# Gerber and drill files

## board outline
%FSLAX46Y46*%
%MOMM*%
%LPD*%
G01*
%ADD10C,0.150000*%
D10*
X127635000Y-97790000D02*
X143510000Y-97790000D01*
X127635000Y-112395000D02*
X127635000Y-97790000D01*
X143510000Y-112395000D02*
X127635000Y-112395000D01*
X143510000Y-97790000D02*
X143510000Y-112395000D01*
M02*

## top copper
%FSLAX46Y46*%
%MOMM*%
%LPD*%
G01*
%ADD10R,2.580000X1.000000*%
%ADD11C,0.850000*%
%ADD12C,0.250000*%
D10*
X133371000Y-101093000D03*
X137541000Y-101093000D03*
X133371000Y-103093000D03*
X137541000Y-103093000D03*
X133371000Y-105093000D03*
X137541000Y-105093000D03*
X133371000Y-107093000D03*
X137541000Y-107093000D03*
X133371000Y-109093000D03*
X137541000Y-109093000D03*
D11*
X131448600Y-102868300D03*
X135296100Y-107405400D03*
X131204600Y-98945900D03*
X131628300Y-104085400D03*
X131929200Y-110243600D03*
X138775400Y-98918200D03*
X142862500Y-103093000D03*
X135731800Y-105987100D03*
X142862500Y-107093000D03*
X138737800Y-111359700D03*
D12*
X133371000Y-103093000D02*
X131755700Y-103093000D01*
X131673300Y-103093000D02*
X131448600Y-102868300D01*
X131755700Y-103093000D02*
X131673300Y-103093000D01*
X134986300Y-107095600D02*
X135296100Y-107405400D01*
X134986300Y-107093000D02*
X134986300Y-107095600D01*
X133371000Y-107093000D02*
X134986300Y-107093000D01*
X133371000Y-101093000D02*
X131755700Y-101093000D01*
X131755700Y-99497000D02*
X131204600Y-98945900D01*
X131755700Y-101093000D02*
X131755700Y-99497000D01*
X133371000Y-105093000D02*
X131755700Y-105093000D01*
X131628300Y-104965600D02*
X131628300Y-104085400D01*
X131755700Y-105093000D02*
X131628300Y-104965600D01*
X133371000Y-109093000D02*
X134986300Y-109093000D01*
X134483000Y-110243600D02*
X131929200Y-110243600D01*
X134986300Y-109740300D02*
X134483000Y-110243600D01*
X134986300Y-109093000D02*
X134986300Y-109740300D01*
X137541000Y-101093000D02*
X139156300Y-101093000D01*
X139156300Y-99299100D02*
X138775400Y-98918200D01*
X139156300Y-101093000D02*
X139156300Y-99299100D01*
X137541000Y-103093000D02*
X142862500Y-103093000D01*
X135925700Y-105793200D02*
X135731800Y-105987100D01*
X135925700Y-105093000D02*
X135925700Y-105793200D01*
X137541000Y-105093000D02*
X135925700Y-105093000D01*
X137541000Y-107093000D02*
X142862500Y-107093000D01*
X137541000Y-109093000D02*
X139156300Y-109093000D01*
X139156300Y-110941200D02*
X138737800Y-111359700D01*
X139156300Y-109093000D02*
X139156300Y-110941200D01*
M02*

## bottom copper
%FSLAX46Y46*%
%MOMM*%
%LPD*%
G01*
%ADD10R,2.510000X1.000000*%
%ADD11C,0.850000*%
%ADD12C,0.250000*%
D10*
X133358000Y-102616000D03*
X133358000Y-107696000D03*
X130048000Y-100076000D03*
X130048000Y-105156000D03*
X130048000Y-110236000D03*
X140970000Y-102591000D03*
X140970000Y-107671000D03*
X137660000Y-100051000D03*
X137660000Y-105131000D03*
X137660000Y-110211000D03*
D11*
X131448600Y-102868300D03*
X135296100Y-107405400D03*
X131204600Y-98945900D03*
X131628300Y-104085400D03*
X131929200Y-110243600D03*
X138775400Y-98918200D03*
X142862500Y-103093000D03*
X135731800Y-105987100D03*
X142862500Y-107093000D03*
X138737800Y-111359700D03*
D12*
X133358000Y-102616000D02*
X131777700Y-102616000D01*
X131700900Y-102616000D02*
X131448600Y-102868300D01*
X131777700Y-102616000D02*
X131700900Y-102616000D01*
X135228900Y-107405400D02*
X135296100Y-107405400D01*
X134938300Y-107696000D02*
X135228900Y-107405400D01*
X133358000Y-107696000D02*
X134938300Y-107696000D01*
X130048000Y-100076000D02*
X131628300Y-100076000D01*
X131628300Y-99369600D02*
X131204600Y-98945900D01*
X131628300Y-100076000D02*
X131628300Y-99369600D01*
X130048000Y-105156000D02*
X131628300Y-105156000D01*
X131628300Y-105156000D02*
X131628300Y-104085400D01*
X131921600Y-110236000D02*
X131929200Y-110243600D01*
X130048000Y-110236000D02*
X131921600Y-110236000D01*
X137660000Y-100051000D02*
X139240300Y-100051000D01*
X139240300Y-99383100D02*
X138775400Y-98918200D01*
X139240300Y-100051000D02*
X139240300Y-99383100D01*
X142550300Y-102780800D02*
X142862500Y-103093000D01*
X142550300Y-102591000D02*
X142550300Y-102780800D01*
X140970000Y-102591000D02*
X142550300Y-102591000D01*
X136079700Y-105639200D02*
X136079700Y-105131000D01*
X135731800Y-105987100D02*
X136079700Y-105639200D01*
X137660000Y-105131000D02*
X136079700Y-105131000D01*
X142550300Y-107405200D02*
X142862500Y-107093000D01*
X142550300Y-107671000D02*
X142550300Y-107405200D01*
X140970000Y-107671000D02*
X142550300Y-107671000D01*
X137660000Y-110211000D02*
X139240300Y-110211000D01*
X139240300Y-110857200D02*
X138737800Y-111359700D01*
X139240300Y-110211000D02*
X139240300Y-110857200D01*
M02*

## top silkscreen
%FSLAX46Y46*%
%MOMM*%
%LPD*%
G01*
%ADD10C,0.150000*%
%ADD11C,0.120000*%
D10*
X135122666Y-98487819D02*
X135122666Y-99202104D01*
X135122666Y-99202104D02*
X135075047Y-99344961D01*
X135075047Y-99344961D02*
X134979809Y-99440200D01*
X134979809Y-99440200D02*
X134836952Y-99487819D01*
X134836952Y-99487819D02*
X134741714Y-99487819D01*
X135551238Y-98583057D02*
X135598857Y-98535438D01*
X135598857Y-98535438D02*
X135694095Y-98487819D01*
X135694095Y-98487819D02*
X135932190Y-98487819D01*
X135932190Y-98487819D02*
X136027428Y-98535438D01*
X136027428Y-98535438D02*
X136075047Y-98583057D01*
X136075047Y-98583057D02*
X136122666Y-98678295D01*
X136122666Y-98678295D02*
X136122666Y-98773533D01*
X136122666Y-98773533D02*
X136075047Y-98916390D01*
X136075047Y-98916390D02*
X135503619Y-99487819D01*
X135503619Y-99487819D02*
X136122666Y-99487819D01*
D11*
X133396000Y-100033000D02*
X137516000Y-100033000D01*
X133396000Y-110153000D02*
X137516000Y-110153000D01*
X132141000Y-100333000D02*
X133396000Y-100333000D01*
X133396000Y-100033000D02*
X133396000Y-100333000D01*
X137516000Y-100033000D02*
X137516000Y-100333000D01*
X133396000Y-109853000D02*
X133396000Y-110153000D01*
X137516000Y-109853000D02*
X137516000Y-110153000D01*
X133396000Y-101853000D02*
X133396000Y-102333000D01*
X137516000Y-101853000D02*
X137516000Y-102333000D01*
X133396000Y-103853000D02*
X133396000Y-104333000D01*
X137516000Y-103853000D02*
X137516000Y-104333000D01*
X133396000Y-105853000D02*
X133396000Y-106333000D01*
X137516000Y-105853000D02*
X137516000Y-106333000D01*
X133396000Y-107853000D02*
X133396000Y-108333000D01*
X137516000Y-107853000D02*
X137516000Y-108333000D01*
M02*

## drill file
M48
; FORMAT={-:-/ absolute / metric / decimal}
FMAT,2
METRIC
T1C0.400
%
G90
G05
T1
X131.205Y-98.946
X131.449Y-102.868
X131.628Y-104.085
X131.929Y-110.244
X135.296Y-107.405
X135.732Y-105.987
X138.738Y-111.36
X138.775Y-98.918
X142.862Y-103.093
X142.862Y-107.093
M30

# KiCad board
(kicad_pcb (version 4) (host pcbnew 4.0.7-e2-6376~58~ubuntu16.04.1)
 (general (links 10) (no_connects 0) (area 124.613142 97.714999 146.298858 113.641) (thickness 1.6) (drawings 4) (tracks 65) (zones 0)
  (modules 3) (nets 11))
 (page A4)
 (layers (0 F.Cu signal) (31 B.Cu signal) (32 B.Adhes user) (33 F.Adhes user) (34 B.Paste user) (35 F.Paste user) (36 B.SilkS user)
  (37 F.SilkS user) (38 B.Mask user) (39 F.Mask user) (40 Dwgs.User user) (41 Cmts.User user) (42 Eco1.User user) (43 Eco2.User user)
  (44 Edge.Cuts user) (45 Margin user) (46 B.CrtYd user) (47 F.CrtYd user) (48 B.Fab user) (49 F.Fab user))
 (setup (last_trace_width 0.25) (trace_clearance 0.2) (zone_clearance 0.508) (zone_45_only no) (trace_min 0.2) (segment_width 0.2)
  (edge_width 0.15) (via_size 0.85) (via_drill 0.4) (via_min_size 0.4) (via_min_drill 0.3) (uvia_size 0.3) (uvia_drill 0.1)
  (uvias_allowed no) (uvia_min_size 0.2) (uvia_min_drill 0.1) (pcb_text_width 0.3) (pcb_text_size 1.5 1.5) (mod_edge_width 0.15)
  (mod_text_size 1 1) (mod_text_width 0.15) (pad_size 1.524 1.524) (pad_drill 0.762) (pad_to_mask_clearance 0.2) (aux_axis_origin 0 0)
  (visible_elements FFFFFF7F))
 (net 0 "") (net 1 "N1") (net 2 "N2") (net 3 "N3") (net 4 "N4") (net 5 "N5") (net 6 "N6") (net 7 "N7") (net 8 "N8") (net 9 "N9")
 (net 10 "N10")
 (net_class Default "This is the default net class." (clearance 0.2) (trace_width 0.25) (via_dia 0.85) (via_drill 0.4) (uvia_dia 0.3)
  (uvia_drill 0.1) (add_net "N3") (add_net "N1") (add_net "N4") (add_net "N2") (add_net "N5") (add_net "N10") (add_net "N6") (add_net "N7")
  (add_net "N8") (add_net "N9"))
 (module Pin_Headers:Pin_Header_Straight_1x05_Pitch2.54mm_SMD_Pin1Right (layer B.Cu) (at 131.703 105.156 180)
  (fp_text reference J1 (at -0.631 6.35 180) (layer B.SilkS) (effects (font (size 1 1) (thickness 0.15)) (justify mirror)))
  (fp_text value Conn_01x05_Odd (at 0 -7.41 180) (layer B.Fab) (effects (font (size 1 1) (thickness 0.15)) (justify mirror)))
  (pad 2 smd rect (at -1.655 2.54 180) (size 2.51 1) (layers B.Cu B.Paste B.Mask) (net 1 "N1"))
  (pad 4 smd rect (at -1.655 -2.54 180) (size 2.51 1) (layers B.Cu B.Paste B.Mask) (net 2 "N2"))
  (pad 1 smd rect (at 1.655 5.08 180) (size 2.51 1) (layers B.Cu B.Paste B.Mask) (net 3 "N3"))
  (pad 3 smd rect (at 1.655 0 180) (size 2.51 1) (layers B.Cu B.Paste B.Mask) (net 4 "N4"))
  (pad 5 smd rect (at 1.655 -5.08 180) (size 2.51 1) (layers B.Cu B.Paste B.Mask) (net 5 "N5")))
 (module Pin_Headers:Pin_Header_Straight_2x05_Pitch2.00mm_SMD (layer F.Cu) (at 135.456 105.093)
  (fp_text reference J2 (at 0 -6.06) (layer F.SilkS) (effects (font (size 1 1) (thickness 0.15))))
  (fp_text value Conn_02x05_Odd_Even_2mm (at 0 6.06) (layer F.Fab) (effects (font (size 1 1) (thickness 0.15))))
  (fp_line (start -2.06 -5.06) (end 2.06 -5.06) (layer F.SilkS) (width 0.12))
  (fp_line (start -2.06 5.06) (end 2.06 5.06) (layer F.SilkS) (width 0.12))
  (fp_line (start -3.315 -4.76) (end -2.06 -4.76) (layer F.SilkS) (width 0.12))
  (fp_line (start -2.06 -5.06) (end -2.06 -4.76) (layer F.SilkS) (width 0.12))
  (fp_line (start 2.06 -5.06) (end 2.06 -4.76) (layer F.SilkS) (width 0.12))
  (fp_line (start -2.06 4.76) (end -2.06 5.06) (layer F.SilkS) (width 0.12))
  (fp_line (start 2.06 4.76) (end 2.06 5.06) (layer F.SilkS) (width 0.12))
  (fp_line (start -2.06 -3.24) (end -2.06 -2.76) (layer F.SilkS) (width 0.12))
  (fp_line (start 2.06 -3.24) (end 2.06 -2.76) (layer F.SilkS) (width 0.12))
  (fp_line (start -2.06 -1.24) (end -2.06 -0.76) (layer F.SilkS) (width 0.12))
  (fp_line (start 2.06 -1.24) (end 2.06 -0.76) (layer F.SilkS) (width 0.12))
  (fp_line (start -2.06 0.76) (end -2.06 1.24) (layer F.SilkS) (width 0.12))
  (fp_line (start 2.06 0.76) (end 2.06 1.24) (layer F.SilkS) (width 0.12))
  (fp_line (start -2.06 2.76) (end -2.06 3.24) (layer F.SilkS) (width 0.12))
  (fp_line (start 2.06 2.76) (end 2.06 3.24) (layer F.SilkS) (width 0.12))
  (pad 1 smd rect (at -2.085 -4) (size 2.58 1) (layers F.Cu F.Paste F.Mask) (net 3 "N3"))
  (pad 2 smd rect (at 2.085 -4) (size 2.58 1) (layers F.Cu F.Paste F.Mask) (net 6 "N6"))
  (pad 3 smd rect (at -2.085 -2) (size 2.58 1) (layers F.Cu F.Paste F.Mask) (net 1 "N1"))
  (pad 4 smd rect (at 2.085 -2) (size 2.58 1) (layers F.Cu F.Paste F.Mask) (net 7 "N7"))
  (pad 5 smd rect (at -2.085 0) (size 2.58 1) (layers F.Cu F.Paste F.Mask) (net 4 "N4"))
  (pad 6 smd rect (at 2.085 0) (size 2.58 1) (layers F.Cu F.Paste F.Mask) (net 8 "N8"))
  (pad 7 smd rect (at -2.085 2) (size 2.58 1) (layers F.Cu F.Paste F.Mask) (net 2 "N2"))
  (pad 8 smd rect (at 2.085 2) (size 2.58 1) (layers F.Cu F.Paste F.Mask) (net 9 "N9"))
  (pad 9 smd rect (at -2.085 4) (size 2.58 1) (layers F.Cu F.Paste F.Mask) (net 5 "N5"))
  (pad 10 smd rect (at 2.085 4) (size 2.58 1) (layers F.Cu F.Paste F.Mask) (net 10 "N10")))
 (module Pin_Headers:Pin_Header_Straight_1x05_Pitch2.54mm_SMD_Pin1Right (layer B.Cu) (at 139.315 105.131 180)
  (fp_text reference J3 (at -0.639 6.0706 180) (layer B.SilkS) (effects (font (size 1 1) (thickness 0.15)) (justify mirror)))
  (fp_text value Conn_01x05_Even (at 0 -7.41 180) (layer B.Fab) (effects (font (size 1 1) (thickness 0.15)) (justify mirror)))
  (pad 2 smd rect (at -1.655 2.54 180) (size 2.51 1) (layers B.Cu B.Paste B.Mask) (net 7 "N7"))
  (pad 4 smd rect (at -1.655 -2.54 180) (size 2.51 1) (layers B.Cu B.Paste B.Mask) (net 9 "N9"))
  (pad 1 smd rect (at 1.655 5.08 180) (size 2.51 1) (layers B.Cu B.Paste B.Mask) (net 6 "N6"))
  (pad 3 smd rect (at 1.655 0 180) (size 2.51 1) (layers B.Cu B.Paste B.Mask) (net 8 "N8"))
  (pad 5 smd rect (at 1.655 -5.08 180) (size 2.51 1) (layers B.Cu B.Paste B.Mask) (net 10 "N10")))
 (gr_line (start 127.635 97.79) (end 143.51 97.79) (layer Edge.Cuts) (width 0.15))
 (gr_line (start 127.635 112.395) (end 127.635 97.79) (layer Edge.Cuts) (width 0.15))
 (gr_line (start 143.51 112.395) (end 127.635 112.395) (layer Edge.Cuts) (width 0.15))
 (gr_line (start 143.51 97.79) (end 143.51 112.395) (layer Edge.Cuts) (width 0.15))
 (via (at 131.4486 102.8683) (size 0.85) (layers F.Cu B.Cu) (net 1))
 (segment (start 133.358 102.616) (end 131.7777 102.616) (width 0.25) (layer B.Cu) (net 1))
 (segment (start 133.371 103.093) (end 131.7557 103.093) (width 0.25) (layer F.Cu) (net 1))
 (segment (start 131.7009 102.616) (end 131.4486 102.8683) (width 0.25) (layer B.Cu) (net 1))
 (segment (start 131.7777 102.616) (end 131.7009 102.616) (width 0.25) (layer B.Cu) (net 1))
 (segment (start 131.6733 103.093) (end 131.4486 102.8683) (width 0.25) (layer F.Cu) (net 1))
 (segment (start 131.7557 103.093) (end 131.6733 103.093) (width 0.25) (layer F.Cu) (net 1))
 (via (at 135.2961 107.4054) (size 0.85) (layers F.Cu B.Cu) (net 2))
 (segment (start 135.2289 107.4054) (end 135.2961 107.4054) (width 0.25) (layer B.Cu) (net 2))
 (segment (start 134.9383 107.696) (end 135.2289 107.4054) (width 0.25) (layer B.Cu) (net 2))
 (segment (start 134.9863 107.0956) (end 135.2961 107.4054) (width 0.25) (layer F.Cu) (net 2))
 (segment (start 134.9863 107.093) (end 134.9863 107.0956) (width 0.25) (layer F.Cu) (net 2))
 (segment (start 133.371 107.093) (end 134.9863 107.093) (width 0.25) (layer F.Cu) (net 2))
 (segment (start 133.358 107.696) (end 134.9383 107.696) (width 0.25) (layer B.Cu) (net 2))
 (via (at 131.2046 98.9459) (size 0.85) (layers F.Cu B.Cu) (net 3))
 (segment (start 133.371 101.093) (end 131.7557 101.093) (width 0.25) (layer F.Cu) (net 3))
 (segment (start 130.048 100.076) (end 131.6283 100.076) (width 0.25) (layer B.Cu) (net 3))
 (segment (start 131.6283 99.3696) (end 131.2046 98.9459) (width 0.25) (layer B.Cu) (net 3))
 (segment (start 131.6283 100.076) (end 131.6283 99.3696) (width 0.25) (layer B.Cu) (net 3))
 (segment (start 131.7557 99.497) (end 131.2046 98.9459) (width 0.25) (layer F.Cu) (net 3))
 (segment (start 131.7557 101.093) (end 131.7557 99.497) (width 0.25) (layer F.Cu) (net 3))
 (via (at 131.6283 104.0854) (size 0.85) (layers F.Cu B.Cu) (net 4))
 (segment (start 133.371 105.093) (end 131.7557 105.093) (width 0.25) (layer F.Cu) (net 4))
 (segment (start 130.048 105.156) (end 131.6283 105.156) (width 0.25) (layer B.Cu) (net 4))
 (segment (start 131.6283 105.156) (end 131.6283 104.0854) (width 0.25) (layer B.Cu) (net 4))
 (segment (start 131.6283 104.9656) (end 131.6283 104.0854) (width 0.25) (layer F.Cu) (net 4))
 (segment (start 131.7557 105.093) (end 131.6283 104.9656) (width 0.25) (layer F.Cu) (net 4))
 (via (at 131.9292 110.2436) (size 0.85) (layers F.Cu B.Cu) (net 5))
 (segment (start 133.371 109.093) (end 134.9863 109.093) (width 0.25) (layer F.Cu) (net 5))
 (segment (start 131.9216 110.236) (end 131.9292 110.2436) (width 0.25) (layer B.Cu) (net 5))
 (segment (start 130.048 110.236) (end 131.9216 110.236) (width 0.25) (layer B.Cu) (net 5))
 (segment (start 134.483 110.2436) (end 131.9292 110.2436) (width 0.25) (layer F.Cu) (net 5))
 (segment (start 134.9863 109.7403) (end 134.483 110.2436) (width 0.25) (layer F.Cu) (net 5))
 (segment (start 134.9863 109.093) (end 134.9863 109.7403) (width 0.25) (layer F.Cu) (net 5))
 (via (at 138.7754 98.9182) (size 0.85) (layers F.Cu B.Cu) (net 6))
 (segment (start 137.541 101.093) (end 139.1563 101.093) (width 0.25) (layer F.Cu) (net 6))
 (segment (start 137.66 100.051) (end 139.2403 100.051) (width 0.25) (layer B.Cu) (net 6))
 (segment (start 139.2403 99.3831) (end 138.7754 98.9182) (width 0.25) (layer B.Cu) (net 6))
 (segment (start 139.2403 100.051) (end 139.2403 99.3831) (width 0.25) (layer B.Cu) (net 6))
 (segment (start 139.1563 99.2991) (end 138.7754 98.9182) (width 0.25) (layer F.Cu) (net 6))
 (segment (start 139.1563 101.093) (end 139.1563 99.2991) (width 0.25) (layer F.Cu) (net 6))
 (via (at 142.8625 103.093) (size 0.85) (layers F.Cu B.Cu) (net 7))
 (segment (start 142.5503 102.7808) (end 142.8625 103.093) (width 0.25) (layer B.Cu) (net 7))
 (segment (start 142.5503 102.591) (end 142.5503 102.7808) (width 0.25) (layer B.Cu) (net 7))
 (segment (start 137.541 103.093) (end 142.8625 103.093) (width 0.25) (layer F.Cu) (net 7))
 (segment (start 140.97 102.591) (end 142.5503 102.591) (width 0.25) (layer B.Cu) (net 7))
 (via (at 135.7318 105.9871) (size 0.85) (layers F.Cu B.Cu) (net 8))
 (segment (start 136.0797 105.6392) (end 136.0797 105.131) (width 0.25) (layer B.Cu) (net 8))
 (segment (start 135.7318 105.9871) (end 136.0797 105.6392) (width 0.25) (layer B.Cu) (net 8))
 (segment (start 135.9257 105.7932) (end 135.7318 105.9871) (width 0.25) (layer F.Cu) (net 8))
 (segment (start 135.9257 105.093) (end 135.9257 105.7932) (width 0.25) (layer F.Cu) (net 8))
 (segment (start 137.66 105.131) (end 136.0797 105.131) (width 0.25) (layer B.Cu) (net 8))
 (segment (start 137.541 105.093) (end 135.9257 105.093) (width 0.25) (layer F.Cu) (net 8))
 (via (at 142.8625 107.093) (size 0.85) (layers F.Cu B.Cu) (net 9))
 (segment (start 142.5503 107.4052) (end 142.8625 107.093) (width 0.25) (layer B.Cu) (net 9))
 (segment (start 142.5503 107.671) (end 142.5503 107.4052) (width 0.25) (layer B.Cu) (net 9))
 (segment (start 137.541 107.093) (end 142.8625 107.093) (width 0.25) (layer F.Cu) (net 9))
 (segment (start 140.97 107.671) (end 142.5503 107.671) (width 0.25) (layer B.Cu) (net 9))
 (via (at 138.7378 111.3597) (size 0.85) (layers F.Cu B.Cu) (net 10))
 (segment (start 137.541 109.093) (end 139.1563 109.093) (width 0.25) (layer F.Cu) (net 10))
 (segment (start 137.66 110.211) (end 139.2403 110.211) (width 0.25) (layer B.Cu) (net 10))
 (segment (start 139.2403 110.8572) (end 138.7378 111.3597) (width 0.25) (layer B.Cu) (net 10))
 (segment (start 139.2403 110.211) (end 139.2403 110.8572) (width 0.25) (layer B.Cu) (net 10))
 (segment (start 139.1563 110.9412) (end 138.7378 111.3597) (width 0.25) (layer F.Cu) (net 10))
 (segment (start 139.1563 109.093) (end 139.1563 110.9412) (width 0.25) (layer F.Cu) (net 10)))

